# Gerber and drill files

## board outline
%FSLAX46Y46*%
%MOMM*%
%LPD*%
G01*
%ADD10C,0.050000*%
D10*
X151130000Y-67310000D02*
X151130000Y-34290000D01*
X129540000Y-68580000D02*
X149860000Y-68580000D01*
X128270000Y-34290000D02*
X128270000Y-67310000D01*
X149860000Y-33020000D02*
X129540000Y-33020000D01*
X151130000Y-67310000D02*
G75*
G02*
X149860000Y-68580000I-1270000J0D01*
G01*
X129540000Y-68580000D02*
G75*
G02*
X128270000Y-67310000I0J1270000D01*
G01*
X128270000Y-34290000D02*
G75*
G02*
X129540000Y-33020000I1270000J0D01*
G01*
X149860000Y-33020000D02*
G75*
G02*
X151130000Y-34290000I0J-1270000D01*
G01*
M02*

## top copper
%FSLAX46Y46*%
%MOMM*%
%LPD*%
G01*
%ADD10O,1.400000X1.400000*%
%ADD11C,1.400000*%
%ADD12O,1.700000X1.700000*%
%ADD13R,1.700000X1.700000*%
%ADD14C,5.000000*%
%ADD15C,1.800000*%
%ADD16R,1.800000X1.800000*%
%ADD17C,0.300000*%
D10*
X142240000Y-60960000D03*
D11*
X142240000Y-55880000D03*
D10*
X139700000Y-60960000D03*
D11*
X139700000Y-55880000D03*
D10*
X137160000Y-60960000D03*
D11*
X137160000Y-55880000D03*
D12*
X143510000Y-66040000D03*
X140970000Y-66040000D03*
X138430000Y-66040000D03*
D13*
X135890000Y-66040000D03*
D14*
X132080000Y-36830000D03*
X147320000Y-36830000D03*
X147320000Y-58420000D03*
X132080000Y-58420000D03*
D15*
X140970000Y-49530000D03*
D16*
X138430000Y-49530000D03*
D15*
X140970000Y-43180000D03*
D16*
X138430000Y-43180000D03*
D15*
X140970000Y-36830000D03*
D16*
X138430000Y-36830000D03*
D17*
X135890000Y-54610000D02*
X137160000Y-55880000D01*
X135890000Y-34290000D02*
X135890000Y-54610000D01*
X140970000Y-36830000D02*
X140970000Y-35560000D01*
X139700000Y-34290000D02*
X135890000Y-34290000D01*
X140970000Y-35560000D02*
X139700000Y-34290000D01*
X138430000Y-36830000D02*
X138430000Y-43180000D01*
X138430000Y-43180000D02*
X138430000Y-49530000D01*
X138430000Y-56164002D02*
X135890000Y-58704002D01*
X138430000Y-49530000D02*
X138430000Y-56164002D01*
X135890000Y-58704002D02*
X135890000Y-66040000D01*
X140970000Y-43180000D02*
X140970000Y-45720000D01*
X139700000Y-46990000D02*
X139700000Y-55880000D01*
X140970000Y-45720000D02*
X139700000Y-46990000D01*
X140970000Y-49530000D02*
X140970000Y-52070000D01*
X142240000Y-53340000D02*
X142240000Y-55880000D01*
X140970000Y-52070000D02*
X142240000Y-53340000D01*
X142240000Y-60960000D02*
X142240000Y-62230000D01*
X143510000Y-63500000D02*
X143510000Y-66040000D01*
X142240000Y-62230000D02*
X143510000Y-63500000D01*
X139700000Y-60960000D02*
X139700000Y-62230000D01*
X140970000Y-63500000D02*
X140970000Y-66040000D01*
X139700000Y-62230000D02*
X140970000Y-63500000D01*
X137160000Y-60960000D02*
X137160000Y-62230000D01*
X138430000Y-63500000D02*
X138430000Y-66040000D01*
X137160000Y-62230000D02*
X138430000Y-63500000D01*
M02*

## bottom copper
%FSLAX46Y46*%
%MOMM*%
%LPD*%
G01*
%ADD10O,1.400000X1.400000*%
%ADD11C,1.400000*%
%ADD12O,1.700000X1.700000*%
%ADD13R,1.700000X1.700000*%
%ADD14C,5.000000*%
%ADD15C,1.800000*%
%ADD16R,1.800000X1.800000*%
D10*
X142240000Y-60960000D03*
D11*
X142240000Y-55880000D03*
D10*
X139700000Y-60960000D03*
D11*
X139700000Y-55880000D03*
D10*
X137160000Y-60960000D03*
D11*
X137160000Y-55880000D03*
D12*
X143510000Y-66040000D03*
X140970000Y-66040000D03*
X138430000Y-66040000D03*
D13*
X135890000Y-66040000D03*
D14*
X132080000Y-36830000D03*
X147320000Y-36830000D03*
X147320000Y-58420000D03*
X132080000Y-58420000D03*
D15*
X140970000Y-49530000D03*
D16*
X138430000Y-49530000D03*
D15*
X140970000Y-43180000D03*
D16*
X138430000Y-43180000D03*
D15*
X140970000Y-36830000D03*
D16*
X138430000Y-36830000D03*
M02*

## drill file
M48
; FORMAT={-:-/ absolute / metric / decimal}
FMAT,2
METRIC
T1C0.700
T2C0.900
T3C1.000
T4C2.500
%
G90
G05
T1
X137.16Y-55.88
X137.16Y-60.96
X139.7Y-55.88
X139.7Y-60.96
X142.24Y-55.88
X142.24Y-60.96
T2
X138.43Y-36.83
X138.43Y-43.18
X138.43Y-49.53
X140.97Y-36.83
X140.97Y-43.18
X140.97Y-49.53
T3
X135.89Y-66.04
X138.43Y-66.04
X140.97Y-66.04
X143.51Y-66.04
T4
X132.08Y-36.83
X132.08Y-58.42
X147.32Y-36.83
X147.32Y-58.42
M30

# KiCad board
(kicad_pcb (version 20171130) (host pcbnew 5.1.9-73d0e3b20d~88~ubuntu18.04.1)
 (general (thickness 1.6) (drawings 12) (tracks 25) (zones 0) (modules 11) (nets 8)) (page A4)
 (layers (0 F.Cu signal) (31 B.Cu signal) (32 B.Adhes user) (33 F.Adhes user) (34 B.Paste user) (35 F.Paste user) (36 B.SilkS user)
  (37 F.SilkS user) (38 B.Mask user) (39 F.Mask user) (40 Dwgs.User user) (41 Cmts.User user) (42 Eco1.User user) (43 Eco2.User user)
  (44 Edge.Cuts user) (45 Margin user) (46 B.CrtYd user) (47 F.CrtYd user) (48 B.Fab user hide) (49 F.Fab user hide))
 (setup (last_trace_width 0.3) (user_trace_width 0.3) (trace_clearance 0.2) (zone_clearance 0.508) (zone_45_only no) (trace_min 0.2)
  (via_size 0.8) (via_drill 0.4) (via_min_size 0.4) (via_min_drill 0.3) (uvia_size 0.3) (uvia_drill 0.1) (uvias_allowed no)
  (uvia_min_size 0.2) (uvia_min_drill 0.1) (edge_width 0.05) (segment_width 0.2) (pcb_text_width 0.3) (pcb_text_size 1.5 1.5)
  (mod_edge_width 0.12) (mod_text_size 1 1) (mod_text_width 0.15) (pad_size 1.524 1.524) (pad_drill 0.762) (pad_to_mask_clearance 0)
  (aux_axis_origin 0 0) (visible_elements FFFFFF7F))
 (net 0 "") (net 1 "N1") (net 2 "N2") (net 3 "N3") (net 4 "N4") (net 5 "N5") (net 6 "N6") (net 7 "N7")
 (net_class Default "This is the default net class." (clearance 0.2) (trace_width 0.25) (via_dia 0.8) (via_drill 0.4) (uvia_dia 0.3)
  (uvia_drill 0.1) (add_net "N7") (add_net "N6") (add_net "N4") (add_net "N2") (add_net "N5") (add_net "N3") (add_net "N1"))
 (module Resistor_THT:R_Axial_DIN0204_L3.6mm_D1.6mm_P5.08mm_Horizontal (layer F.Cu) (at 142.24 55.88 270)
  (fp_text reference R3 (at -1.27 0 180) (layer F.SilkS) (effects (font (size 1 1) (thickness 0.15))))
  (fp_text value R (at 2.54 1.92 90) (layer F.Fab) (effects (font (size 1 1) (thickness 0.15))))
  (pad 2 thru_hole oval (at 5.08 0 270) (size 1.4 1.4) (drill 0.7) (layers *.Cu *.Mask) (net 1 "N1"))
  (pad 1 thru_hole circle (at 0 0 270) (size 1.4 1.4) (drill 0.7) (layers *.Cu *.Mask) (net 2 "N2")))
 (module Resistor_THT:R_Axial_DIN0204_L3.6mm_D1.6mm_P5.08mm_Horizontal (layer F.Cu) (at 139.7 55.88 270)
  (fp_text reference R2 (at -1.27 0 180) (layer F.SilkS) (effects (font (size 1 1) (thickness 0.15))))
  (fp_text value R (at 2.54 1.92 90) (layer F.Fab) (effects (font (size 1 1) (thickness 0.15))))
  (pad 2 thru_hole oval (at 5.08 0 270) (size 1.4 1.4) (drill 0.7) (layers *.Cu *.Mask) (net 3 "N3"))
  (pad 1 thru_hole circle (at 0 0 270) (size 1.4 1.4) (drill 0.7) (layers *.Cu *.Mask) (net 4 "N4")))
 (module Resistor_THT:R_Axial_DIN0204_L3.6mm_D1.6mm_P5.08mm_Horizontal (layer F.Cu) (at 137.16 55.88 270)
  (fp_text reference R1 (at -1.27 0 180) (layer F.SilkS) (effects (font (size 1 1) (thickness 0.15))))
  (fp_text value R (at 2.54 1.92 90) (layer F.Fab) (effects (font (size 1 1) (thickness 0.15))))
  (pad 2 thru_hole oval (at 5.08 0 270) (size 1.4 1.4) (drill 0.7) (layers *.Cu *.Mask) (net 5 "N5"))
  (pad 1 thru_hole circle (at 0 0 270) (size 1.4 1.4) (drill 0.7) (layers *.Cu *.Mask) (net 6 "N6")))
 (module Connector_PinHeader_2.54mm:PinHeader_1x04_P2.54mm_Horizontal (layer B.Cu) (at 135.89 66.04 270)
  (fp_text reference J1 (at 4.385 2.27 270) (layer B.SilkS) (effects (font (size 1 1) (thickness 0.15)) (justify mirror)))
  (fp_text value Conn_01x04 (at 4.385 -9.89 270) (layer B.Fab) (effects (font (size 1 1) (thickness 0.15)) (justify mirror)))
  (pad 4 thru_hole oval (at 0 -7.62 270) (size 1.7 1.7) (drill 1) (layers *.Cu *.Mask) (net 1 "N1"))
  (pad 3 thru_hole oval (at 0 -5.08 270) (size 1.7 1.7) (drill 1) (layers *.Cu *.Mask) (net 3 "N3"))
  (pad 2 thru_hole oval (at 0 -2.54 270) (size 1.7 1.7) (drill 1) (layers *.Cu *.Mask) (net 5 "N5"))
  (pad 1 thru_hole rect (at 0 0 270) (size 1.7 1.7) (drill 1) (layers *.Cu *.Mask) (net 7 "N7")))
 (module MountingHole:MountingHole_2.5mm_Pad (layer F.Cu) (at 132.08 36.83)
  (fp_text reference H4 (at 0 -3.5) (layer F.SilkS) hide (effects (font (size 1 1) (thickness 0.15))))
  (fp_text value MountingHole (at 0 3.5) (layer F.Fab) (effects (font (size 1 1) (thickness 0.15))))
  (pad 1 thru_hole circle (at 0 0) (size 5 5) (drill 2.5) (layers *.Cu *.Mask)))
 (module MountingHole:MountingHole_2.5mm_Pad (layer F.Cu) (at 147.32 36.83)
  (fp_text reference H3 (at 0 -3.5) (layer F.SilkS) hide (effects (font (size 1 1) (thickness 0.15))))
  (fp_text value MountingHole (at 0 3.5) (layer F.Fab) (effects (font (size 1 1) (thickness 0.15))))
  (pad 1 thru_hole circle (at 0 0) (size 5 5) (drill 2.5) (layers *.Cu *.Mask)))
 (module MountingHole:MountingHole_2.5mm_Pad (layer F.Cu) (at 147.32 58.42)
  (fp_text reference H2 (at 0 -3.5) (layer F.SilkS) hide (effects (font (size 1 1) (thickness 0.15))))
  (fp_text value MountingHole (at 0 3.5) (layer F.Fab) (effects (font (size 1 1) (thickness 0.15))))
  (pad 1 thru_hole circle (at 0 0) (size 5 5) (drill 2.5) (layers *.Cu *.Mask)))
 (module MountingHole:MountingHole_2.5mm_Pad (layer F.Cu) (at 132.08 58.42)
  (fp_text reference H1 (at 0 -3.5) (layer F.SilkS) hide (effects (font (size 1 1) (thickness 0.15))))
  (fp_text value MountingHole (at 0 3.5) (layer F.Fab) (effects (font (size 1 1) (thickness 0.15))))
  (pad 1 thru_hole circle (at 0 0) (size 5 5) (drill 2.5) (layers *.Cu *.Mask)))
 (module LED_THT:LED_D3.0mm (layer F.Cu) (at 138.43 49.53)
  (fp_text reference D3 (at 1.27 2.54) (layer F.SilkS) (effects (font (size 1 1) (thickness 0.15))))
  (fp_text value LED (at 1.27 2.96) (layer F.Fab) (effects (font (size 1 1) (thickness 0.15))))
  (pad 2 thru_hole circle (at 2.54 0) (size 1.8 1.8) (drill 0.9) (layers *.Cu *.Mask) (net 2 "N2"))
  (pad 1 thru_hole rect (at 0 0) (size 1.8 1.8) (drill 0.9) (layers *.Cu *.Mask) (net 7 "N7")))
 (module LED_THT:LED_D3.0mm (layer F.Cu) (at 138.43 43.18)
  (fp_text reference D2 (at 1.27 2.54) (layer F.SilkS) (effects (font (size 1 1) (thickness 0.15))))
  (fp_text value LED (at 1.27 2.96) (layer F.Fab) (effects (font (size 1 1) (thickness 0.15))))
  (pad 2 thru_hole circle (at 2.54 0) (size 1.8 1.8) (drill 0.9) (layers *.Cu *.Mask) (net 4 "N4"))
  (pad 1 thru_hole rect (at 0 0) (size 1.8 1.8) (drill 0.9) (layers *.Cu *.Mask) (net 7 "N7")))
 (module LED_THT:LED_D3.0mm (layer F.Cu) (at 138.43 36.83)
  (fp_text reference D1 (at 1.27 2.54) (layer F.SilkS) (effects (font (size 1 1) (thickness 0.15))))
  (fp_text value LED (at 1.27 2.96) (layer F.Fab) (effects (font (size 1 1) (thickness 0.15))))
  (pad 2 thru_hole circle (at 2.54 0) (size 1.8 1.8) (drill 0.9) (layers *.Cu *.Mask) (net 6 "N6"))
  (pad 1 thru_hole rect (at 0 0) (size 1.8 1.8) (drill 0.9) (layers *.Cu *.Mask) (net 7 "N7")))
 (gr_line (start 151.13 67.31) (end 151.13 34.29) (layer Edge.Cuts) (width 0.05))
 (gr_line (start 129.54 68.58) (end 149.86 68.58) (layer Edge.Cuts) (width 0.05))
 (gr_line (start 128.27 34.29) (end 128.27 67.31) (layer Edge.Cuts) (width 0.05))
 (gr_line (start 149.86 33.02) (end 129.54 33.02) (layer Edge.Cuts) (width 0.05))
 (gr_arc (start 149.86 67.31) (end 149.86 68.58) (angle -90) (layer Edge.Cuts) (width 0.05))
 (gr_arc (start 129.54 67.31) (end 128.27 67.31) (angle -90) (layer Edge.Cuts) (width 0.05))
 (gr_arc (start 129.54 34.29) (end 129.54 33.02) (angle -90) (layer Edge.Cuts) (width 0.05))
 (gr_arc (start 149.86 34.29) (end 151.13 34.29) (angle -90) (layer Edge.Cuts) (width 0.05))
 (segment (start 135.89 54.61) (end 137.16 55.88) (width 0.3) (layer F.Cu) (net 6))
 (segment (start 135.89 34.29) (end 135.89 54.61) (width 0.3) (layer F.Cu) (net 6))
 (segment (start 140.97 36.83) (end 140.97 35.56) (width 0.3) (layer F.Cu) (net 6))
 (segment (start 139.7 34.29) (end 135.89 34.29) (width 0.3) (layer F.Cu) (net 6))
 (segment (start 140.97 35.56) (end 139.7 34.29) (width 0.3) (layer F.Cu) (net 6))
 (segment (start 138.43 36.83) (end 138.43 43.18) (width 0.3) (layer F.Cu) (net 7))
 (segment (start 138.43 43.18) (end 138.43 49.53) (width 0.3) (layer F.Cu) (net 7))
 (segment (start 138.43 56.164002) (end 135.89 58.704002) (width 0.3) (layer F.Cu) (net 7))
 (segment (start 138.43 49.53) (end 138.43 56.164002) (width 0.3) (layer F.Cu) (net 7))
 (segment (start 135.89 58.704002) (end 135.89 66.04) (width 0.3) (layer F.Cu) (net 7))
 (segment (start 140.97 43.18) (end 140.97 45.72) (width 0.3) (layer F.Cu) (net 4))
 (segment (start 139.7 46.99) (end 139.7 55.88) (width 0.3) (layer F.Cu) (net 4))
 (segment (start 140.97 45.72) (end 139.7 46.99) (width 0.3) (layer F.Cu) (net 4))
 (segment (start 140.97 49.53) (end 140.97 52.07) (width 0.3) (layer F.Cu) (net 2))
 (segment (start 142.24 53.34) (end 142.24 55.88) (width 0.3) (layer F.Cu) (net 2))
 (segment (start 140.97 52.07) (end 142.24 53.34) (width 0.3) (layer F.Cu) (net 2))
 (segment (start 142.24 60.96) (end 142.24 62.23) (width 0.3) (layer F.Cu) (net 1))
 (segment (start 143.51 63.5) (end 143.51 66.04) (width 0.3) (layer F.Cu) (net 1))
 (segment (start 142.24 62.23) (end 143.51 63.5) (width 0.3) (layer F.Cu) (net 1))
 (segment (start 139.7 60.96) (end 139.7 62.23) (width 0.3) (layer F.Cu) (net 3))
 (segment (start 140.97 63.5) (end 140.97 66.04) (width 0.3) (layer F.Cu) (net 3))
 (segment (start 139.7 62.23) (end 140.97 63.5) (width 0.3) (layer F.Cu) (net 3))
 (segment (start 137.16 60.96) (end 137.16 62.23) (width 0.3) (layer F.Cu) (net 5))
 (segment (start 138.43 63.5) (end 138.43 66.04) (width 0.3) (layer F.Cu) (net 5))
 (segment (start 137.16 62.23) (end 138.43 63.5) (width 0.3) (layer F.Cu) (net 5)))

